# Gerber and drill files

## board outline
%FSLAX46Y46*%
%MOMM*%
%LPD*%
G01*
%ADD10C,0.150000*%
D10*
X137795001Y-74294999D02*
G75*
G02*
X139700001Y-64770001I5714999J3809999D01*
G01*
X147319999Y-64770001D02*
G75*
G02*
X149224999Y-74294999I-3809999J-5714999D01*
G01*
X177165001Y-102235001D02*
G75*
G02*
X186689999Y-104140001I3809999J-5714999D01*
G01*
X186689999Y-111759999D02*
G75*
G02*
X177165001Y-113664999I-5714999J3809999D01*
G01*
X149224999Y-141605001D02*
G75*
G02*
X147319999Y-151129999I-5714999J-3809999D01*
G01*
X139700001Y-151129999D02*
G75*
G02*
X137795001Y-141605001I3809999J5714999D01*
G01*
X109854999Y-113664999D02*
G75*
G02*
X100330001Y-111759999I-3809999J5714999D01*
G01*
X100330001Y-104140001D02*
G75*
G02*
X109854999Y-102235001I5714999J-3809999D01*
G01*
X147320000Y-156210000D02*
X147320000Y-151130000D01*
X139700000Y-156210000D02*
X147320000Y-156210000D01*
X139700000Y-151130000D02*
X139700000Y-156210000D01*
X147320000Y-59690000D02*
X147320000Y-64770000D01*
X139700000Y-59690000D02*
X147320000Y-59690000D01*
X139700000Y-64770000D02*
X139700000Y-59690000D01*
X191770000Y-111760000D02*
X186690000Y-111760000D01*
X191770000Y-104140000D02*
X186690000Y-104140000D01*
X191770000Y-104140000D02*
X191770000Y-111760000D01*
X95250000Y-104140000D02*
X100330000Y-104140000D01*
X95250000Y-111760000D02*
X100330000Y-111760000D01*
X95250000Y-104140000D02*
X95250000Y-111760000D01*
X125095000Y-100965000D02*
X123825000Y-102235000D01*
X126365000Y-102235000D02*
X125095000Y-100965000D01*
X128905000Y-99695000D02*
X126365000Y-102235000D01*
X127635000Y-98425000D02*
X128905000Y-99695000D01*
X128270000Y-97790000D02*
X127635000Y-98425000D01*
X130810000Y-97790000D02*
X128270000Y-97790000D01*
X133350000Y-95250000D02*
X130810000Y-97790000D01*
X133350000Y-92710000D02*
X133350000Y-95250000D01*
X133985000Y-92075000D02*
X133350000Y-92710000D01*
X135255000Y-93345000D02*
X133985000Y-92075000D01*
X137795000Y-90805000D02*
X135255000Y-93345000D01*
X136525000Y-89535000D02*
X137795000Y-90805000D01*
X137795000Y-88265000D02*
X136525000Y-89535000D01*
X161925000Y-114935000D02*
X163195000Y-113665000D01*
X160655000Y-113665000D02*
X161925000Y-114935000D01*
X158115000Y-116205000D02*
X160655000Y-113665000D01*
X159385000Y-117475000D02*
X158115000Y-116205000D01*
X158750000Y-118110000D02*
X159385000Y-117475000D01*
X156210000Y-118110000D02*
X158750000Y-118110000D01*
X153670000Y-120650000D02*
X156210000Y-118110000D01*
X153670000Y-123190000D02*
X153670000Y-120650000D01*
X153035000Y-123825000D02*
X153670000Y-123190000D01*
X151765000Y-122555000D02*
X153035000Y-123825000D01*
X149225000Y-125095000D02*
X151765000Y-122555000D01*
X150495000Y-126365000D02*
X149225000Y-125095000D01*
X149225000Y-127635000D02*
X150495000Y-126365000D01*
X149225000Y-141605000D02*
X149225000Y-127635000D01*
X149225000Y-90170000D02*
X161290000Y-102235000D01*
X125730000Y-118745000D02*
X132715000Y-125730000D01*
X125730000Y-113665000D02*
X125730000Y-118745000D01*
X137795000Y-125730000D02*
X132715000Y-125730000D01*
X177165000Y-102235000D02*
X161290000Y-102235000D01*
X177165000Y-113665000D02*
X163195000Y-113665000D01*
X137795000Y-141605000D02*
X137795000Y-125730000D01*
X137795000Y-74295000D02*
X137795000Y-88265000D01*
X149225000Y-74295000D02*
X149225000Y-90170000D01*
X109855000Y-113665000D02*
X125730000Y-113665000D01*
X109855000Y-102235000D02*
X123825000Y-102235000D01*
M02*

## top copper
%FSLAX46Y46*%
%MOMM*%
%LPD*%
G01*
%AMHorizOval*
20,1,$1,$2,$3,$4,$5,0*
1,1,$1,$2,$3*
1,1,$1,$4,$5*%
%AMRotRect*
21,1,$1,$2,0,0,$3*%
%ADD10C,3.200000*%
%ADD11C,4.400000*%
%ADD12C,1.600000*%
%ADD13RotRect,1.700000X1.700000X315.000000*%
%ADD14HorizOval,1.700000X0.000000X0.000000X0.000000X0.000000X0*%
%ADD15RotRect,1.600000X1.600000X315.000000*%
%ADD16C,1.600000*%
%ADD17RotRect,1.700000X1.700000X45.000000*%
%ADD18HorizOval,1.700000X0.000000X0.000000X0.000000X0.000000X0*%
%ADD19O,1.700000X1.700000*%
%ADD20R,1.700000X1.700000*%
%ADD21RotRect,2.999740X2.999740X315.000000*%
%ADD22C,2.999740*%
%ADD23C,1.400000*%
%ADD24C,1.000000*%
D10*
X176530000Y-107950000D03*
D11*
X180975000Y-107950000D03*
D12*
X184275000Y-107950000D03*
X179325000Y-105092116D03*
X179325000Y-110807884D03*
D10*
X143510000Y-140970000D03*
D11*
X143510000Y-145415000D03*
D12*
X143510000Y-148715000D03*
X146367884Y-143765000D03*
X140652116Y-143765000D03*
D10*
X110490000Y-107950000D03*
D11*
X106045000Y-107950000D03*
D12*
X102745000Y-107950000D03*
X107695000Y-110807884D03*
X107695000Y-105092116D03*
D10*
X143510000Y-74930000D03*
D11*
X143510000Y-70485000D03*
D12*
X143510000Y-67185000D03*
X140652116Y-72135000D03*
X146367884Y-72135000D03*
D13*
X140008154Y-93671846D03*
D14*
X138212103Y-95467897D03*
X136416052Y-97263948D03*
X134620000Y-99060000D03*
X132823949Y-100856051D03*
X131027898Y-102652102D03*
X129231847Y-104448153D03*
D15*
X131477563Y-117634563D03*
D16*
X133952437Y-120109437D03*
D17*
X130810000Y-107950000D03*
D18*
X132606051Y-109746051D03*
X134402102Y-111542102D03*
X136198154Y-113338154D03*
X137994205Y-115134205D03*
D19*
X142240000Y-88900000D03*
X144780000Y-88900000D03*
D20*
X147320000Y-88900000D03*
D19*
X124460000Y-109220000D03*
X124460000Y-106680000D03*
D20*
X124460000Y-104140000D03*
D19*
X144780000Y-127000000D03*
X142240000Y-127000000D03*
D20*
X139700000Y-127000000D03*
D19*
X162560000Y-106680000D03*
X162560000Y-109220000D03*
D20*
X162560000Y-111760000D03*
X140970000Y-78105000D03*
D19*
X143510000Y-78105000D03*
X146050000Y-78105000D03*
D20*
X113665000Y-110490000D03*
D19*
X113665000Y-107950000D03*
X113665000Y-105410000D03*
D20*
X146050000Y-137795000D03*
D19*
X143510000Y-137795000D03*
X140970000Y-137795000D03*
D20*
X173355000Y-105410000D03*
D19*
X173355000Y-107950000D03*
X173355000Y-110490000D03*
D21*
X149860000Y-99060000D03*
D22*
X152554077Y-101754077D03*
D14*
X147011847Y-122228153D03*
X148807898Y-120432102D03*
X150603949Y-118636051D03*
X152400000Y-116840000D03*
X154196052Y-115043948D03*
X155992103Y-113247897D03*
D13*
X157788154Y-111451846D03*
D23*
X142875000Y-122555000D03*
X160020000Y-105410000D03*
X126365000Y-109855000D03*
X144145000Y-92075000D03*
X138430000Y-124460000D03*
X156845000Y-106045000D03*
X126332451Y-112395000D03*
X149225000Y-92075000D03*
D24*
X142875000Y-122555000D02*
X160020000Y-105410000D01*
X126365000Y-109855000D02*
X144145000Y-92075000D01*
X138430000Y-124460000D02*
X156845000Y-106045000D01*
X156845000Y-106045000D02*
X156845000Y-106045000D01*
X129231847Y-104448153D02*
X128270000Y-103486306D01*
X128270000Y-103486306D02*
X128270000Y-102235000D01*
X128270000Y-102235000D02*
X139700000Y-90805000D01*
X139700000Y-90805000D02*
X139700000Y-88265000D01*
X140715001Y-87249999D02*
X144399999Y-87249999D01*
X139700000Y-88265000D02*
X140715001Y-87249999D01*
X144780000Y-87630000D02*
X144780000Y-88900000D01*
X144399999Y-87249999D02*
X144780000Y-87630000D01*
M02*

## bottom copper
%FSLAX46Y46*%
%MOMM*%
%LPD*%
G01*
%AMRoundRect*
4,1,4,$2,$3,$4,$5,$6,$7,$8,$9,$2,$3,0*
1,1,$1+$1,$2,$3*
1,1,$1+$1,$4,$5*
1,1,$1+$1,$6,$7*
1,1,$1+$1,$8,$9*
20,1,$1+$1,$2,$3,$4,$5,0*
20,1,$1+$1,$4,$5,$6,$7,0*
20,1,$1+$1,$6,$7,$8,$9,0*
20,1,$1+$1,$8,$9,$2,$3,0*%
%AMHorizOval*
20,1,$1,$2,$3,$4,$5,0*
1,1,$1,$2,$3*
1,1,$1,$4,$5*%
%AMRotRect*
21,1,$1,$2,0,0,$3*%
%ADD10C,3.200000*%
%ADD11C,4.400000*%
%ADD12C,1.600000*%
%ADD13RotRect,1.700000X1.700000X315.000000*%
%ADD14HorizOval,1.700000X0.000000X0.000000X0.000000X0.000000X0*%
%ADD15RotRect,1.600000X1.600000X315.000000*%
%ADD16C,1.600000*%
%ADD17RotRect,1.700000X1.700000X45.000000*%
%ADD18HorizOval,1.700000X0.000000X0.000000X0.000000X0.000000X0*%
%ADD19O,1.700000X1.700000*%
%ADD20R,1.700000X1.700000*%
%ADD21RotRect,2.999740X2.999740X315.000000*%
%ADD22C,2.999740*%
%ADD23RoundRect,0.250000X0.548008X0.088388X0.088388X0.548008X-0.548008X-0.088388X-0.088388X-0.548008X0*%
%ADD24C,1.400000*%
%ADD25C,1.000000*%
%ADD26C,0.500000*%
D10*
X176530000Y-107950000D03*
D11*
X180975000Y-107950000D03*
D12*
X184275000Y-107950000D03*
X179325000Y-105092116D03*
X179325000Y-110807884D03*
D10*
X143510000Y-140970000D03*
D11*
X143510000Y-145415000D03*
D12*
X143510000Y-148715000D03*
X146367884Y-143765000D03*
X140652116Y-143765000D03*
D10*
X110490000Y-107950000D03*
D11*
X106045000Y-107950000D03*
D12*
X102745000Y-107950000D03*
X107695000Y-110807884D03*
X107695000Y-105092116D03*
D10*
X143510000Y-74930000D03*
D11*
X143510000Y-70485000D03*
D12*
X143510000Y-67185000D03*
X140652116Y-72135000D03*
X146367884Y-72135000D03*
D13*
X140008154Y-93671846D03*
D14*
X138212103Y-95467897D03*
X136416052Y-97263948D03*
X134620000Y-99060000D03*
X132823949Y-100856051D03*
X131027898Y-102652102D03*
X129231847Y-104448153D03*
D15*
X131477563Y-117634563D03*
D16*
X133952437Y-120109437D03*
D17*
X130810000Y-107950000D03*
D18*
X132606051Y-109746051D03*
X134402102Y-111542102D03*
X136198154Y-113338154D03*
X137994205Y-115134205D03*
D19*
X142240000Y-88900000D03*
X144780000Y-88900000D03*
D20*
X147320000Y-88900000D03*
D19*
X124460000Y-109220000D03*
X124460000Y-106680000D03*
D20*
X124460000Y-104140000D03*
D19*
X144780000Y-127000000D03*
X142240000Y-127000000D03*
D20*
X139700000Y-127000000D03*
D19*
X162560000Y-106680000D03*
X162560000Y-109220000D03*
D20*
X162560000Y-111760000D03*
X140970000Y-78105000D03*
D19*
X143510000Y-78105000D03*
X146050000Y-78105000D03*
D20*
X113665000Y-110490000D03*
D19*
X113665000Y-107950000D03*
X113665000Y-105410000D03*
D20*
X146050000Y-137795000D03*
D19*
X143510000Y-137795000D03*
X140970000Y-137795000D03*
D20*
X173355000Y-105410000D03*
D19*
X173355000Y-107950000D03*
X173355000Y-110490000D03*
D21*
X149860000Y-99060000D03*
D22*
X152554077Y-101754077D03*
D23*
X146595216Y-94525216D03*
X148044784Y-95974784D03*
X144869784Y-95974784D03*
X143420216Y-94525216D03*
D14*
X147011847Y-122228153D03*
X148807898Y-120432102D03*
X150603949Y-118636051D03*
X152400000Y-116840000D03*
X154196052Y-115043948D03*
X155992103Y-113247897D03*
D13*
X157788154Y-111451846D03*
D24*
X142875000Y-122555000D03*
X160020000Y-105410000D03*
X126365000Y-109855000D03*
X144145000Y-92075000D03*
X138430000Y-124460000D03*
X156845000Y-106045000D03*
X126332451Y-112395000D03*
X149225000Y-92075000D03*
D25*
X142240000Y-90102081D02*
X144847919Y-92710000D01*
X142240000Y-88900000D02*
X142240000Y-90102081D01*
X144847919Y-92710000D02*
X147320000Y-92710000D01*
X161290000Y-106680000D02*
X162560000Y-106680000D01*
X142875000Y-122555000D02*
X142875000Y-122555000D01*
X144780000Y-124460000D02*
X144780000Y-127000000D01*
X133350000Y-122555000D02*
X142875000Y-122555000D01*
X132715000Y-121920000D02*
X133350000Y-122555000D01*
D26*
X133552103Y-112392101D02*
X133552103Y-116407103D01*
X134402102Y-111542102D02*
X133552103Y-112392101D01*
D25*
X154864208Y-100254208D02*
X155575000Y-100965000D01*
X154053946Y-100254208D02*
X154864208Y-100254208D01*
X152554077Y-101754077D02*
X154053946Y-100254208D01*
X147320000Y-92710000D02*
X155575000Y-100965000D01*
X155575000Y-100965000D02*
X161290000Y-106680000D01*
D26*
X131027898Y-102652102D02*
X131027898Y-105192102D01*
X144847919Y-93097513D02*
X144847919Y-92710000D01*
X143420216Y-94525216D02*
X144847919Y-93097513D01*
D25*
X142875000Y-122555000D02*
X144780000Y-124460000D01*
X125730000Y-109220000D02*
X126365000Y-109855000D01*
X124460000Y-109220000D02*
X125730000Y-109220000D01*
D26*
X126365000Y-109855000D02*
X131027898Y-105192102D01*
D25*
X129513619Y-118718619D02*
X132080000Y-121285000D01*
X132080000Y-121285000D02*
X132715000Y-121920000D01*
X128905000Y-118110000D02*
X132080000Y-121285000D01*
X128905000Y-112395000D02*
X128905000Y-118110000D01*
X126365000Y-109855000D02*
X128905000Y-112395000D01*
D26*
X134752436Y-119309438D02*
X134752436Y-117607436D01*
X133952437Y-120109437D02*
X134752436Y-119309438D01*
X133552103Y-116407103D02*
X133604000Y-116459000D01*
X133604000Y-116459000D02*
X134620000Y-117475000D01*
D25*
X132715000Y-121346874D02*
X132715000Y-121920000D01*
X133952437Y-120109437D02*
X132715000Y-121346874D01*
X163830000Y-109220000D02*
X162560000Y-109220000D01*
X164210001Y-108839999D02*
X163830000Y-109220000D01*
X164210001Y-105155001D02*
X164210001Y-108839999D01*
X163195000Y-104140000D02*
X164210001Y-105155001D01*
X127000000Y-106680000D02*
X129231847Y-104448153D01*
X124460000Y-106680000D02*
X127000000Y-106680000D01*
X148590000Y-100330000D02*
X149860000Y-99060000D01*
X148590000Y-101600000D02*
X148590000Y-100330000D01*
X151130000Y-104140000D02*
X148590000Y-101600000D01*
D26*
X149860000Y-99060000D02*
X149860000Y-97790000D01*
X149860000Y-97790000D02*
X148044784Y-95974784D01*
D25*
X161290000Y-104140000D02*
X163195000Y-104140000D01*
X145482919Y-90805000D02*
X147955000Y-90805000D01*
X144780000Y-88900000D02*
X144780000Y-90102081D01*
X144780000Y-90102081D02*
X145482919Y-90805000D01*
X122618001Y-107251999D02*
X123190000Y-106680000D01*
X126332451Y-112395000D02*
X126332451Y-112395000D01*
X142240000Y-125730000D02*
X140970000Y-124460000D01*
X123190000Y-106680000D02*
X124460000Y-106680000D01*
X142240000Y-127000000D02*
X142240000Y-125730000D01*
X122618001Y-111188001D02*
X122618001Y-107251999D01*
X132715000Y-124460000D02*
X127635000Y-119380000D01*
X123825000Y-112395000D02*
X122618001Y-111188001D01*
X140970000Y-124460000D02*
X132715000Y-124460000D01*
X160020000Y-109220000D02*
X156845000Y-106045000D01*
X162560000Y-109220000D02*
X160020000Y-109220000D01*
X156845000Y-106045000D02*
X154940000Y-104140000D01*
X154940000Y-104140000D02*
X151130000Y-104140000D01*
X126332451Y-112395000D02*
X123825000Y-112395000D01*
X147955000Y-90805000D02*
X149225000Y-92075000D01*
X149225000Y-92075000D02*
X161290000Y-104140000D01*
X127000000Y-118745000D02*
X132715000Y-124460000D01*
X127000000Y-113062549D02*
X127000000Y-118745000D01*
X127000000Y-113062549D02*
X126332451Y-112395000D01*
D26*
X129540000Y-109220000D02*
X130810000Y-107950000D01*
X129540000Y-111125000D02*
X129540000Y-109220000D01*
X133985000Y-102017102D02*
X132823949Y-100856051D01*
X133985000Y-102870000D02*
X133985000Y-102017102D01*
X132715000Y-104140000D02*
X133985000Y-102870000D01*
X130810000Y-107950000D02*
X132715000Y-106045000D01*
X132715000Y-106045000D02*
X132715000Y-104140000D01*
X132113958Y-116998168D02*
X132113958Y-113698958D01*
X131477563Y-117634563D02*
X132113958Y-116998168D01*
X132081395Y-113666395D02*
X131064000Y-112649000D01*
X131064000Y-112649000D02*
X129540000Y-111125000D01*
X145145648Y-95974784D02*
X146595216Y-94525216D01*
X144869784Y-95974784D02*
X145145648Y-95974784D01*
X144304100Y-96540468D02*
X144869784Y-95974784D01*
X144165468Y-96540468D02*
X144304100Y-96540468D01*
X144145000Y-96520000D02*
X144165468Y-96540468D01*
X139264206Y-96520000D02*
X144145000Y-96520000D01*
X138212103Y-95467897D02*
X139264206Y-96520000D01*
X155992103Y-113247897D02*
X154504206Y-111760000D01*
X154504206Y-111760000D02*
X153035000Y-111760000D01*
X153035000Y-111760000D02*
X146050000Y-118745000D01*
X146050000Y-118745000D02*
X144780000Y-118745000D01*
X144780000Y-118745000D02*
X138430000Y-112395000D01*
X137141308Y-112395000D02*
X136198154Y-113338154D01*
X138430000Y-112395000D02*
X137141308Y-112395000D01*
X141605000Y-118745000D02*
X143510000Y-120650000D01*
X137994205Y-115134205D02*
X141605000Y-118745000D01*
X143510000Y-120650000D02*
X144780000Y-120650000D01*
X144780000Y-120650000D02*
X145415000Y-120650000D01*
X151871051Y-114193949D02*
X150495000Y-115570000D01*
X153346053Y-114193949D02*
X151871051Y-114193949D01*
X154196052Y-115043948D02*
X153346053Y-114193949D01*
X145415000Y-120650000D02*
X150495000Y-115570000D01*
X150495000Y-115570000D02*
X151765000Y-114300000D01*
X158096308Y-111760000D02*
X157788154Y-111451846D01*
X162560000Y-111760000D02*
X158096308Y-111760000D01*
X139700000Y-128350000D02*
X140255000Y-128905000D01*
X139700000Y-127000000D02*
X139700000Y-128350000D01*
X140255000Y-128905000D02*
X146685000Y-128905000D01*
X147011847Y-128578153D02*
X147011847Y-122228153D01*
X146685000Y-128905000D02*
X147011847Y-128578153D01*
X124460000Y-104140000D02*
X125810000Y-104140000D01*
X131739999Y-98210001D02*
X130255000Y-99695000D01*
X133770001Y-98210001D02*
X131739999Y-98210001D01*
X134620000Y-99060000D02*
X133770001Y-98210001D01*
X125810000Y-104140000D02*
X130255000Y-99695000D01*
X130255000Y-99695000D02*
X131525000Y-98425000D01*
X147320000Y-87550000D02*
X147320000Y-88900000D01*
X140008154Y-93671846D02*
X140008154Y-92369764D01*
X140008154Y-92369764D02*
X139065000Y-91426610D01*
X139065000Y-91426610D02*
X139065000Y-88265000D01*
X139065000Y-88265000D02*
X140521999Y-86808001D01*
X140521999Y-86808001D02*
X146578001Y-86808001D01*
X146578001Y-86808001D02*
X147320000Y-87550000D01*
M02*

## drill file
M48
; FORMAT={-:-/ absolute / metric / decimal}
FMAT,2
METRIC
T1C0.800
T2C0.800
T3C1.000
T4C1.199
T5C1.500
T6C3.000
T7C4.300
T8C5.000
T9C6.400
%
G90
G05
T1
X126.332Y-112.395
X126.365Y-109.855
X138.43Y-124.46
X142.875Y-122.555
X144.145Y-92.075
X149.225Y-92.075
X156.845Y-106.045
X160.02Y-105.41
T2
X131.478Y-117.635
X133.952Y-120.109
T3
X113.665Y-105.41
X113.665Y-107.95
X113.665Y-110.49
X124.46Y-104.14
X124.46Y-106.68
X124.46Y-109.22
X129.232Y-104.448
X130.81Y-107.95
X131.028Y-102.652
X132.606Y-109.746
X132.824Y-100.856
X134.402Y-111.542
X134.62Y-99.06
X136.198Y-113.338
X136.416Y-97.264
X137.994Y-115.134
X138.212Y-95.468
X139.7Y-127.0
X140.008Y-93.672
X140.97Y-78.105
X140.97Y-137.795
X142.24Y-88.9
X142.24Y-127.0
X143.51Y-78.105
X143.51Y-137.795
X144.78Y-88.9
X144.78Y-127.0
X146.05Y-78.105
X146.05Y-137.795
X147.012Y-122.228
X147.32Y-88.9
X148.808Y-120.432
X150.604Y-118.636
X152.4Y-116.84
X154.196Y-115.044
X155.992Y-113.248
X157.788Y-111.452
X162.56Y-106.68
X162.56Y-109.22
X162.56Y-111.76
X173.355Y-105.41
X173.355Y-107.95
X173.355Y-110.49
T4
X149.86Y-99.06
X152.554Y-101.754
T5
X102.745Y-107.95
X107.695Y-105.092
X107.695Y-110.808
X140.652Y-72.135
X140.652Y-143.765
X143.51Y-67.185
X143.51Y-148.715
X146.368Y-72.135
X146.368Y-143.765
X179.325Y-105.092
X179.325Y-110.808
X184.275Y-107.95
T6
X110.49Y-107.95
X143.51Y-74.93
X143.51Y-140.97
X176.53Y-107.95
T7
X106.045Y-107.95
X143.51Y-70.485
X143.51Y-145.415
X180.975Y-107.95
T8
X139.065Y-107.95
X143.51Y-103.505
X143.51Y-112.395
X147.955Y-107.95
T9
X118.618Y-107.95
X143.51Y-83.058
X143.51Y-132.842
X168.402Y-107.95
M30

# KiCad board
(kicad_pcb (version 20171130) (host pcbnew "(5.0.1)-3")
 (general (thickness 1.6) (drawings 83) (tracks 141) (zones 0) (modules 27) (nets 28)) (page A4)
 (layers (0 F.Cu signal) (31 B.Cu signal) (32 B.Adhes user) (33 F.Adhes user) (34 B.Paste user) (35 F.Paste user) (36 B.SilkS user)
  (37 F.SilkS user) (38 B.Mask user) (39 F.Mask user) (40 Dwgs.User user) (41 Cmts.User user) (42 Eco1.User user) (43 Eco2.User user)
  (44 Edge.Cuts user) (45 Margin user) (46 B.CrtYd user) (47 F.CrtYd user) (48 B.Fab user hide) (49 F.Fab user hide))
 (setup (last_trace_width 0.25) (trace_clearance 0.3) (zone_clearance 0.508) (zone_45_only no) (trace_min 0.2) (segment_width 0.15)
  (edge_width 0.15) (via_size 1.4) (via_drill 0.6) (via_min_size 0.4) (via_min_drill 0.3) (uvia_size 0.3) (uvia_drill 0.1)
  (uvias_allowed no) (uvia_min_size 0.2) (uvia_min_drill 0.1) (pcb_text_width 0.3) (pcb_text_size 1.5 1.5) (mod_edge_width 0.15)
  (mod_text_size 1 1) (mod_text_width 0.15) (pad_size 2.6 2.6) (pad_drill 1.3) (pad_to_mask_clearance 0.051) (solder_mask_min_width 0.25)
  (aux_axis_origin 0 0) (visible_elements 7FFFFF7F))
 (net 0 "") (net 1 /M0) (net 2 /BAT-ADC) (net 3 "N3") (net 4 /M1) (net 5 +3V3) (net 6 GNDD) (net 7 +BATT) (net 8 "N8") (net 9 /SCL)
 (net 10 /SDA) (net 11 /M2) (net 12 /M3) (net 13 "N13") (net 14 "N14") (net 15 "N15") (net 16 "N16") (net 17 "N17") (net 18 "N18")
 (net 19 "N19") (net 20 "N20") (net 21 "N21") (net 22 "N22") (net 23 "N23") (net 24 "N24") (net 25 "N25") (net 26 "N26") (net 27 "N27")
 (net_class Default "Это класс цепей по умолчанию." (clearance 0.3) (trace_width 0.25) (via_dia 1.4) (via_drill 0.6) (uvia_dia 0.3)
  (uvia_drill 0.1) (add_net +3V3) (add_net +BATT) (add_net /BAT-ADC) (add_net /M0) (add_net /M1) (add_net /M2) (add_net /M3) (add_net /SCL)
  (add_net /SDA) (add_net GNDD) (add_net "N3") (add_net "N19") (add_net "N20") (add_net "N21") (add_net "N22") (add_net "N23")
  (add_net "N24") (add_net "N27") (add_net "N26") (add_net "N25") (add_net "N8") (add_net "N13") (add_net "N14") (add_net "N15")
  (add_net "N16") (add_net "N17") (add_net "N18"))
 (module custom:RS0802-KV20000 (layer F.Cu) (at 180.975 107.95)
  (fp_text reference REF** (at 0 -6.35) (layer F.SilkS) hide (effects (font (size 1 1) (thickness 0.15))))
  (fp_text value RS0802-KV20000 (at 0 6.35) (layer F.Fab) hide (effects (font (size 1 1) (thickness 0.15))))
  (pad "" np_thru_hole circle (at -4.445 0) (size 3.2 3.2) (drill 3) (layers *.Cu *.Mask))
  (pad "" np_thru_hole circle (at 0 0) (size 4.4 4.4) (drill 4.3) (layers *.Cu *.Mask))
  (pad "" np_thru_hole circle (at 3.3 0) (size 1.6 1.6) (drill 1.5) (layers *.Cu *.Mask))
  (pad "" np_thru_hole circle (at -1.65 -2.857884 120) (size 1.6 1.6) (drill 1.5) (layers *.Cu *.Mask))
  (pad "" np_thru_hole circle (at -1.65 2.857884 240) (size 1.6 1.6) (drill 1.5) (layers *.Cu *.Mask)))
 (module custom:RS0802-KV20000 (layer F.Cu) (at 143.51 145.415 270)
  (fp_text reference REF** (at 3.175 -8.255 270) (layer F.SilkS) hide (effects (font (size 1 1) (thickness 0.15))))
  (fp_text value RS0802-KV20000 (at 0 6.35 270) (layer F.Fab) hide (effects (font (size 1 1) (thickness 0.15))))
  (pad "" np_thru_hole circle (at -4.445 0 270) (size 3.2 3.2) (drill 3) (layers *.Cu *.Mask))
  (pad "" np_thru_hole circle (at 0 0 270) (size 4.4 4.4) (drill 4.3) (layers *.Cu *.Mask))
  (pad "" np_thru_hole circle (at 3.3 0 270) (size 1.6 1.6) (drill 1.5) (layers *.Cu *.Mask))
  (pad "" np_thru_hole circle (at -1.65 -2.857884 30) (size 1.6 1.6) (drill 1.5) (layers *.Cu *.Mask))
  (pad "" np_thru_hole circle (at -1.65 2.857884 150) (size 1.6 1.6) (drill 1.5) (layers *.Cu *.Mask)))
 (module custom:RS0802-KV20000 (layer F.Cu) (at 106.045 107.95 180)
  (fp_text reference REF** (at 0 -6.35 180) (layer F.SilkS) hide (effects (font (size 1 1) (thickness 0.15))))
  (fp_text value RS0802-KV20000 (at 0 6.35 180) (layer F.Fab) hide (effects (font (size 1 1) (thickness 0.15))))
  (pad "" np_thru_hole circle (at -4.445 0 180) (size 3.2 3.2) (drill 3) (layers *.Cu *.Mask))
  (pad "" np_thru_hole circle (at 0 0 180) (size 4.4 4.4) (drill 4.3) (layers *.Cu *.Mask))
  (pad "" np_thru_hole circle (at 3.3 0 180) (size 1.6 1.6) (drill 1.5) (layers *.Cu *.Mask))
  (pad "" np_thru_hole circle (at -1.65 -2.857884 300) (size 1.6 1.6) (drill 1.5) (layers *.Cu *.Mask))
  (pad "" np_thru_hole circle (at -1.65 2.857884 60) (size 1.6 1.6) (drill 1.5) (layers *.Cu *.Mask)))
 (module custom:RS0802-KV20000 (layer F.Cu) (at 143.51 70.485 90)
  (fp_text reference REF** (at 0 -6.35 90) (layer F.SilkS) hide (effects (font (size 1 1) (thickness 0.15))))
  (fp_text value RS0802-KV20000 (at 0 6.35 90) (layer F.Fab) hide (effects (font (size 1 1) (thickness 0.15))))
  (pad "" np_thru_hole circle (at -4.445 0 90) (size 3.2 3.2) (drill 3) (layers *.Cu *.Mask))
  (pad "" np_thru_hole circle (at 0 0 90) (size 4.4 4.4) (drill 4.3) (layers *.Cu *.Mask))
  (pad "" np_thru_hole circle (at 3.3 0 90) (size 1.6 1.6) (drill 1.5) (layers *.Cu *.Mask))
  (pad "" np_thru_hole circle (at -1.65 -2.857884 210) (size 1.6 1.6) (drill 1.5) (layers *.Cu *.Mask))
  (pad "" np_thru_hole circle (at -1.65 2.857884 330) (size 1.6 1.6) (drill 1.5) (layers *.Cu *.Mask)))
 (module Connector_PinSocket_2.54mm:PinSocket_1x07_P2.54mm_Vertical (layer F.Cu) (at 140.008154 93.671846 315)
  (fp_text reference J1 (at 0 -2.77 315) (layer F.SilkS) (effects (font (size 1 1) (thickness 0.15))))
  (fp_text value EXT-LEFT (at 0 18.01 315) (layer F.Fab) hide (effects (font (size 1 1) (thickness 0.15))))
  (pad 1 thru_hole rect (at 0 0 315) (size 1.7 1.7) (drill 1) (layers *.Cu *.Mask) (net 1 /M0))
  (pad 2 thru_hole oval (at 0 2.54 315) (size 1.7 1.7) (drill 1) (layers *.Cu *.Mask) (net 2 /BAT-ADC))
  (pad 3 thru_hole oval (at 0 5.079999 315) (size 1.7 1.7) (drill 1) (layers *.Cu *.Mask) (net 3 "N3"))
  (pad 4 thru_hole oval (at 0 7.62 315) (size 1.7 1.7) (drill 1) (layers *.Cu *.Mask) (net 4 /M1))
  (pad 5 thru_hole oval (at 0 10.16 315) (size 1.7 1.7) (drill 1) (layers *.Cu *.Mask) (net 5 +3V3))
  (pad 6 thru_hole oval (at 0 12.7 315) (size 1.7 1.7) (drill 1) (layers *.Cu *.Mask) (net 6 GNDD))
  (pad 7 thru_hole oval (at 0 15.24 315) (size 1.7 1.7) (drill 1) (layers *.Cu *.Mask) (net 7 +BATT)))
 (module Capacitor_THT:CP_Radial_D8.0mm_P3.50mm (layer F.Cu) (at 132.715 118.872 315)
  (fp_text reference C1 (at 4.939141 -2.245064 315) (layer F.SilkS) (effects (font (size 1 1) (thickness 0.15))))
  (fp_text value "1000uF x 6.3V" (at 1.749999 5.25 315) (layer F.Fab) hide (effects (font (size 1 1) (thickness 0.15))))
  (pad 1 thru_hole rect (at -1.75 0 315) (size 1.6 1.6) (drill 0.8) (layers *.Cu *.Mask) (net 5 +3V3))
  (pad 2 thru_hole circle (at 1.75 0 315) (size 1.6 1.6) (drill 0.8) (layers *.Cu *.Mask) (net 6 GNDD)))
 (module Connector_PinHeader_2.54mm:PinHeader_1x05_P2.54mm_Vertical (layer F.Cu) (at 130.81 107.95 45)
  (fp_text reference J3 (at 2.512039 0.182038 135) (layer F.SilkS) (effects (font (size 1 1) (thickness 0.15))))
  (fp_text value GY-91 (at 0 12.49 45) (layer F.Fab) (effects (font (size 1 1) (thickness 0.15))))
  (pad 1 thru_hole rect (at 0 0 45) (size 1.7 1.7) (drill 1) (layers *.Cu *.Mask) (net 5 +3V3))
  (pad 2 thru_hole oval (at 0 2.54 45) (size 1.7 1.7) (drill 1) (layers *.Cu *.Mask) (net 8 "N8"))
  (pad 3 thru_hole oval (at 0 5.079999 45) (size 1.7 1.7) (drill 1) (layers *.Cu *.Mask) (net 6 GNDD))
  (pad 4 thru_hole oval (at 0 7.62 45) (size 1.7 1.7) (drill 1) (layers *.Cu *.Mask) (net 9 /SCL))
  (pad 5 thru_hole oval (at 0 10.16 45) (size 1.7 1.7) (drill 1) (layers *.Cu *.Mask) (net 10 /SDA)))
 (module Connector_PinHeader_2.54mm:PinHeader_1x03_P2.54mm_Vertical (layer F.Cu) (at 147.32 88.9 270)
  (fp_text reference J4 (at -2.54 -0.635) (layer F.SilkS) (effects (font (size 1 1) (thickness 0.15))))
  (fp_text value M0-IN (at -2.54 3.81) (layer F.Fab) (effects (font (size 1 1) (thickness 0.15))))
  (pad 3 thru_hole oval (at 0 5.08 270) (size 1.7 1.7) (drill 1) (layers *.Cu *.Mask) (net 6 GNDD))
  (pad 2 thru_hole oval (at 0 2.54 270) (size 1.7 1.7) (drill 1) (layers *.Cu *.Mask) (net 7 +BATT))
  (pad 1 thru_hole rect (at 0 0 270) (size 1.7 1.7) (drill 1) (layers *.Cu *.Mask) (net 1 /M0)))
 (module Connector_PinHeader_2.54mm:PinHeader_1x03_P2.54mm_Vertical (layer F.Cu) (at 124.46 104.14)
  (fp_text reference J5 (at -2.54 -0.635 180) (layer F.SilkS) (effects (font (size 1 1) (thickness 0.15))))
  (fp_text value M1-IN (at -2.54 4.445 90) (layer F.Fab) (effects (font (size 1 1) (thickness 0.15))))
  (pad 3 thru_hole oval (at 0 5.08) (size 1.7 1.7) (drill 1) (layers *.Cu *.Mask) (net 6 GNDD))
  (pad 2 thru_hole oval (at 0 2.54) (size 1.7 1.7) (drill 1) (layers *.Cu *.Mask) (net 7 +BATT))
  (pad 1 thru_hole rect (at 0 0) (size 1.7 1.7) (drill 1) (layers *.Cu *.Mask) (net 4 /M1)))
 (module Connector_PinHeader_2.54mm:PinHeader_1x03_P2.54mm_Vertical (layer F.Cu) (at 139.7 127 90)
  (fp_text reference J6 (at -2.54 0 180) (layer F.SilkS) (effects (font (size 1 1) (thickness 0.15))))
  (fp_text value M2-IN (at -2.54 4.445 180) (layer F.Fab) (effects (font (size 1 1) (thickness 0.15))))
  (pad 3 thru_hole oval (at 0 5.08 90) (size 1.7 1.7) (drill 1) (layers *.Cu *.Mask) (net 6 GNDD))
  (pad 2 thru_hole oval (at 0 2.54 90) (size 1.7 1.7) (drill 1) (layers *.Cu *.Mask) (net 7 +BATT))
  (pad 1 thru_hole rect (at 0 0 90) (size 1.7 1.7) (drill 1) (layers *.Cu *.Mask) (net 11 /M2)))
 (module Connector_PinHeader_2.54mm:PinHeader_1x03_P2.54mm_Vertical (layer F.Cu) (at 162.56 111.76 180)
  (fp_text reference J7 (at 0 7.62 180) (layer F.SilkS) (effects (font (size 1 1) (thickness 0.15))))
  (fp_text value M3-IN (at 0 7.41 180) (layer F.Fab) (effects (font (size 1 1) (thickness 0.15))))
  (pad 3 thru_hole oval (at 0 5.08 180) (size 1.7 1.7) (drill 1) (layers *.Cu *.Mask) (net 6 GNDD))
  (pad 2 thru_hole oval (at 0 2.54 180) (size 1.7 1.7) (drill 1) (layers *.Cu *.Mask) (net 7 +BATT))
  (pad 1 thru_hole rect (at 0 0 180) (size 1.7 1.7) (drill 1) (layers *.Cu *.Mask) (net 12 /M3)))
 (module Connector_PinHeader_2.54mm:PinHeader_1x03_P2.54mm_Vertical (layer F.Cu) (at 140.97 78.105 90)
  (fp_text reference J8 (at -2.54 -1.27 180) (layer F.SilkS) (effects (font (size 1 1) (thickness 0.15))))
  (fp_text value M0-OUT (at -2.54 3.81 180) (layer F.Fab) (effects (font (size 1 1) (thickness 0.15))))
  (pad 1 thru_hole rect (at 0 0 90) (size 1.7 1.7) (drill 1) (layers *.Cu *.Mask) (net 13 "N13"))
  (pad 2 thru_hole oval (at 0 2.54 90) (size 1.7 1.7) (drill 1) (layers *.Cu *.Mask) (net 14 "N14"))
  (pad 3 thru_hole oval (at 0 5.08 90) (size 1.7 1.7) (drill 1) (layers *.Cu *.Mask) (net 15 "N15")))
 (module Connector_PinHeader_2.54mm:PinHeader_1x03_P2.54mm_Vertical (layer F.Cu) (at 113.665 110.49 180)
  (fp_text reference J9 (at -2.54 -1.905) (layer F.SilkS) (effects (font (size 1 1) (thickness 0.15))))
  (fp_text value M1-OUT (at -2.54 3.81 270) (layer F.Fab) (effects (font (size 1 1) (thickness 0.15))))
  (pad 1 thru_hole rect (at 0 0 180) (size 1.7 1.7) (drill 1) (layers *.Cu *.Mask) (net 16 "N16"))
  (pad 2 thru_hole oval (at 0 2.54 180) (size 1.7 1.7) (drill 1) (layers *.Cu *.Mask) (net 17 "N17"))
  (pad 3 thru_hole oval (at 0 5.08 180) (size 1.7 1.7) (drill 1) (layers *.Cu *.Mask) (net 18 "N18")))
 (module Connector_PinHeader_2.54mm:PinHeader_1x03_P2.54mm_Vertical (layer F.Cu) (at 146.05 137.795 270)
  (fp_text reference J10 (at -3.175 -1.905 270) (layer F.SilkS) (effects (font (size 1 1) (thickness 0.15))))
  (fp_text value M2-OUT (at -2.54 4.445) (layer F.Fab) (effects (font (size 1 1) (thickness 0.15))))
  (pad 1 thru_hole rect (at 0 0 270) (size 1.7 1.7) (drill 1) (layers *.Cu *.Mask) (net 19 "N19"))
  (pad 2 thru_hole oval (at 0 2.54 270) (size 1.7 1.7) (drill 1) (layers *.Cu *.Mask) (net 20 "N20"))
  (pad 3 thru_hole oval (at 0 5.08 270) (size 1.7 1.7) (drill 1) (layers *.Cu *.Mask) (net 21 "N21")))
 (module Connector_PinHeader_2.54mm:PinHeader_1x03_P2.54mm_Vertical (layer F.Cu) (at 173.355 105.41)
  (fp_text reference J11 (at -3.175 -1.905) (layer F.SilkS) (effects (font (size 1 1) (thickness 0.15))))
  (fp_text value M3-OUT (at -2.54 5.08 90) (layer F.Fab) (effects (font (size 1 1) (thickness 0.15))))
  (pad 1 thru_hole rect (at 0 0) (size 1.7 1.7) (drill 1) (layers *.Cu *.Mask) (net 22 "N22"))
  (pad 2 thru_hole oval (at 0 2.54) (size 1.7 1.7) (drill 1) (layers *.Cu *.Mask) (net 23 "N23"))
  (pad 3 thru_hole oval (at 0 5.08) (size 1.7 1.7) (drill 1) (layers *.Cu *.Mask) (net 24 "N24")))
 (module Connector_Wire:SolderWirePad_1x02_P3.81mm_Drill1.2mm (layer F.Cu) (at 149.86 99.06 315)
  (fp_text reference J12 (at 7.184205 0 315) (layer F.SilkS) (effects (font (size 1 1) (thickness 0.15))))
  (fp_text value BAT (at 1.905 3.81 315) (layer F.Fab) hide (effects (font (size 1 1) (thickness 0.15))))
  (pad 1 thru_hole rect (at 0 0 315) (size 2.99974 2.99974) (drill 1.19888) (layers *.Cu *.Mask) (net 7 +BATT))
  (pad 2 thru_hole circle (at 3.81 0 315) (size 2.99974 2.99974) (drill 1.19888) (layers *.Cu *.Mask) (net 6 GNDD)))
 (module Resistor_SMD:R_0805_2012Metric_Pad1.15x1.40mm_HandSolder (layer B.Cu) (at 147.32 95.25 135)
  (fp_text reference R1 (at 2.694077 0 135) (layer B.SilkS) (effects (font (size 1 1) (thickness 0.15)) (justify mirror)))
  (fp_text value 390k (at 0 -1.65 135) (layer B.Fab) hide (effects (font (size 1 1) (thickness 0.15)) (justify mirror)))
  (pad 2 smd roundrect (at 1.024999 0 135) (size 1.15 1.4) (layers B.Cu B.Paste B.Mask) (roundrect_rratio 0.217391) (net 2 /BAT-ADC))
  (pad 1 smd roundrect (at -1.024999 0 135) (size 1.15 1.4) (layers B.Cu B.Paste B.Mask) (roundrect_rratio 0.217391) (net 7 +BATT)))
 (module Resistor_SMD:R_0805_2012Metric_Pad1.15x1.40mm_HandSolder (layer B.Cu) (at 144.145 95.25 135)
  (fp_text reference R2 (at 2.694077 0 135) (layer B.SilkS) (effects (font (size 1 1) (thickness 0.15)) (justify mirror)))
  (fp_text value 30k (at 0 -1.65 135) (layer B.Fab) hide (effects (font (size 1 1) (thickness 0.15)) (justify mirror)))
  (pad 1 smd roundrect (at -1.024999 0 135) (size 1.15 1.4) (layers B.Cu B.Paste B.Mask) (roundrect_rratio 0.217391) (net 2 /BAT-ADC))
  (pad 2 smd roundrect (at 1.024999 0 135) (size 1.15 1.4) (layers B.Cu B.Paste B.Mask) (roundrect_rratio 0.217391) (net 6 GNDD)))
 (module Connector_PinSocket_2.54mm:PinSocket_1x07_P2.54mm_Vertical (layer F.Cu) (at 157.788154 111.451846 315)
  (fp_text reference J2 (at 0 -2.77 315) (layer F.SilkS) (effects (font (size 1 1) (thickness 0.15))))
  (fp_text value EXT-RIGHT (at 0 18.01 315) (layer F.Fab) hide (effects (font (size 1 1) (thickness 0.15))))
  (pad 7 thru_hole oval (at 0 15.24 315) (size 1.7 1.7) (drill 1) (layers *.Cu *.Mask) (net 11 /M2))
  (pad 6 thru_hole oval (at 0 12.7 315) (size 1.7 1.7) (drill 1) (layers *.Cu *.Mask) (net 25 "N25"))
  (pad 5 thru_hole oval (at 0 10.16 315) (size 1.7 1.7) (drill 1) (layers *.Cu *.Mask) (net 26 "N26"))
  (pad 4 thru_hole oval (at 0 7.62 315) (size 1.7 1.7) (drill 1) (layers *.Cu *.Mask) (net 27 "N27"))
  (pad 3 thru_hole oval (at 0 5.079999 315) (size 1.7 1.7) (drill 1) (layers *.Cu *.Mask) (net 10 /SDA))
  (pad 2 thru_hole oval (at 0 2.54 315) (size 1.7 1.7) (drill 1) (layers *.Cu *.Mask) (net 9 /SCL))
  (pad 1 thru_hole rect (at 0 0 315) (size 1.7 1.7) (drill 1) (layers *.Cu *.Mask) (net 12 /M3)))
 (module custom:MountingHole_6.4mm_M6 (layer F.Cu) (at 118.618 107.95)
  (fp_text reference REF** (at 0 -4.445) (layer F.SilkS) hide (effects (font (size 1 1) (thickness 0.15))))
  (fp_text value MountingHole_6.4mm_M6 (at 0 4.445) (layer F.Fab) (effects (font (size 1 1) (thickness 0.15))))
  (pad 1 np_thru_hole circle (at 0 0) (size 6.4 6.4) (drill 6.4) (layers *.Cu *.Mask)))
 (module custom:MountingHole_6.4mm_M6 (layer F.Cu) (at 143.51 132.842)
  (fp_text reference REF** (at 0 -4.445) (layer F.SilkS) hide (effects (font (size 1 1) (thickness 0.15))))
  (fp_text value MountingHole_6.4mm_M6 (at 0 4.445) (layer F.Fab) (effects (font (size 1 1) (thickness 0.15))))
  (pad 1 np_thru_hole circle (at 0 0) (size 6.4 6.4) (drill 6.4) (layers *.Cu *.Mask)))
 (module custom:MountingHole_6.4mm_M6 (layer F.Cu) (at 168.402 107.95)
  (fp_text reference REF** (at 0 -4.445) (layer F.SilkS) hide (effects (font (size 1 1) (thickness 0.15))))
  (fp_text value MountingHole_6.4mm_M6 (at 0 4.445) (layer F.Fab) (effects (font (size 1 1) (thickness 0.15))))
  (pad 1 np_thru_hole circle (at 0 0) (size 6.4 6.4) (drill 6.4) (layers *.Cu *.Mask)))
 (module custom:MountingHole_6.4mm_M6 (layer F.Cu) (at 143.51 83.058)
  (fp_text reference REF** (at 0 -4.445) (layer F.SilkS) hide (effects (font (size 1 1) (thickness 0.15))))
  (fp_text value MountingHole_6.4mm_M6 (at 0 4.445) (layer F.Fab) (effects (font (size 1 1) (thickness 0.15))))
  (pad 1 np_thru_hole circle (at 0 0) (size 6.4 6.4) (drill 6.4) (layers *.Cu *.Mask)))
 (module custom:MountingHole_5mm (layer F.Cu) (at 143.51 112.395)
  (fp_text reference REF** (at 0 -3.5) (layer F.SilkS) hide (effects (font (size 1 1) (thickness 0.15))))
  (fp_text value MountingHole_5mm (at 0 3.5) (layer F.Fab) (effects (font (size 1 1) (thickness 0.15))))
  (pad "" np_thru_hole circle (at 0 0) (size 5 5) (drill 5) (layers *.Cu *.Mask)))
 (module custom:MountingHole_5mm (layer F.Cu) (at 139.065 107.95)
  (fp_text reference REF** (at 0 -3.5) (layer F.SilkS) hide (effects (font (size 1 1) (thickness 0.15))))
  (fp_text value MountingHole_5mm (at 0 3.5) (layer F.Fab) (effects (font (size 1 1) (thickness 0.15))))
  (pad "" np_thru_hole circle (at 0 0) (size 5 5) (drill 5) (layers *.Cu *.Mask)))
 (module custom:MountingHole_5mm (layer F.Cu) (at 143.51 103.505)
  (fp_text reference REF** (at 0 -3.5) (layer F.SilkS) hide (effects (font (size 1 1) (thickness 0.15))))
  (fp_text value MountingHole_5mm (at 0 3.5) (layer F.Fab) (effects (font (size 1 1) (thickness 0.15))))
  (pad "" np_thru_hole circle (at 0 0) (size 5 5) (drill 5) (layers *.Cu *.Mask)))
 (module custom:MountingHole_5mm (layer F.Cu) (at 147.955 107.95)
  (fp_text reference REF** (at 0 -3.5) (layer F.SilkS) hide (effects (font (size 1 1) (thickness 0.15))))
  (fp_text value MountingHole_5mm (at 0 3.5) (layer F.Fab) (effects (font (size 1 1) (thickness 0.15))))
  (pad "" np_thru_hole circle (at 0 0) (size 5 5) (drill 5) (layers *.Cu *.Mask)))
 (gr_arc (start 143.51 70.485) (end 139.700001 64.770001) (angle -90) (layer Edge.Cuts) (width 0.15))
 (gr_arc (start 143.51 70.485) (end 149.224999 74.294999) (angle -90) (layer Edge.Cuts) (width 0.15))
 (gr_arc (start 180.975 107.95) (end 186.689999 104.140001) (angle -90) (layer Edge.Cuts) (width 0.15))
 (gr_arc (start 180.975 107.95) (end 177.165001 113.664999) (angle -90) (layer Edge.Cuts) (width 0.15))
 (gr_arc (start 143.51 145.415) (end 147.319999 151.129999) (angle -90) (layer Edge.Cuts) (width 0.15))
 (gr_arc (start 143.51 145.415) (end 137.795001 141.605001) (angle -90) (layer Edge.Cuts) (width 0.15))
 (gr_arc (start 106.045 107.95) (end 100.330001 111.759999) (angle -90) (layer Edge.Cuts) (width 0.15))
 (gr_arc (start 106.045 107.95) (end 109.854999 102.235001) (angle -90) (layer Edge.Cuts) (width 0.15))
 (gr_line (start 147.32 156.21) (end 147.32 151.13) (layer Edge.Cuts) (width 0.15))
 (gr_line (start 139.7 156.21) (end 147.32 156.21) (layer Edge.Cuts) (width 0.15))
 (gr_line (start 139.7 151.13) (end 139.7 156.21) (layer Edge.Cuts) (width 0.15))
 (gr_line (start 147.32 59.69) (end 147.32 64.77) (layer Edge.Cuts) (width 0.15))
 (gr_line (start 139.7 59.69) (end 147.32 59.69) (layer Edge.Cuts) (width 0.15))
 (gr_line (start 139.7 64.77) (end 139.7 59.69) (layer Edge.Cuts) (width 0.15))
 (gr_line (start 191.77 111.76) (end 186.69 111.76) (layer Edge.Cuts) (width 0.15))
 (gr_line (start 191.77 104.14) (end 186.69 104.14) (layer Edge.Cuts) (width 0.15))
 (gr_line (start 191.77 104.14) (end 191.77 111.76) (layer Edge.Cuts) (width 0.15))
 (gr_line (start 95.25 104.14) (end 100.33 104.14) (layer Edge.Cuts) (width 0.15))
 (gr_line (start 95.25 111.76) (end 100.33 111.76) (layer Edge.Cuts) (width 0.15))
 (gr_line (start 95.25 104.14) (end 95.25 111.76) (layer Edge.Cuts) (width 0.15))
 (gr_line (start 125.095 100.965) (end 123.825 102.235) (layer Edge.Cuts) (width 0.15))
 (gr_line (start 126.365 102.235) (end 125.095 100.965) (layer Edge.Cuts) (width 0.15))
 (gr_line (start 128.905 99.695) (end 126.365 102.235) (layer Edge.Cuts) (width 0.15))
 (gr_line (start 127.635 98.425) (end 128.905 99.695) (layer Edge.Cuts) (width 0.15))
 (gr_line (start 128.27 97.79) (end 127.635 98.425) (layer Edge.Cuts) (width 0.15))
 (gr_line (start 130.81 97.79) (end 128.27 97.79) (layer Edge.Cuts) (width 0.15))
 (gr_line (start 133.35 95.25) (end 130.81 97.79) (layer Edge.Cuts) (width 0.15))
 (gr_line (start 133.35 92.71) (end 133.35 95.25) (layer Edge.Cuts) (width 0.15))
 (gr_line (start 133.985 92.075) (end 133.35 92.71) (layer Edge.Cuts) (width 0.15))
 (gr_line (start 135.255 93.345) (end 133.985 92.075) (layer Edge.Cuts) (width 0.15))
 (gr_line (start 137.795 90.805) (end 135.255 93.345) (layer Edge.Cuts) (width 0.15))
 (gr_line (start 136.525 89.535) (end 137.795 90.805) (layer Edge.Cuts) (width 0.15))
 (gr_line (start 137.795 88.265) (end 136.525 89.535) (layer Edge.Cuts) (width 0.15))
 (gr_line (start 161.925 114.935) (end 163.195 113.665) (layer Edge.Cuts) (width 0.15))
 (gr_line (start 160.655 113.665) (end 161.925 114.935) (layer Edge.Cuts) (width 0.15))
 (gr_line (start 158.115 116.205) (end 160.655 113.665) (layer Edge.Cuts) (width 0.15))
 (gr_line (start 159.385 117.475) (end 158.115 116.205) (layer Edge.Cuts) (width 0.15))
 (gr_line (start 158.75 118.11) (end 159.385 117.475) (layer Edge.Cuts) (width 0.15))
 (gr_line (start 156.21 118.11) (end 158.75 118.11) (layer Edge.Cuts) (width 0.15))
 (gr_line (start 153.67 120.65) (end 156.21 118.11) (layer Edge.Cuts) (width 0.15))
 (gr_line (start 153.67 123.19) (end 153.67 120.65) (layer Edge.Cuts) (width 0.15))
 (gr_line (start 153.035 123.825) (end 153.67 123.19) (layer Edge.Cuts) (width 0.15))
 (gr_line (start 151.765 122.555) (end 153.035 123.825) (layer Edge.Cuts) (width 0.15))
 (gr_line (start 149.225 125.095) (end 151.765 122.555) (layer Edge.Cuts) (width 0.15))
 (gr_line (start 150.495 126.365) (end 149.225 125.095) (layer Edge.Cuts) (width 0.15))
 (gr_line (start 149.225 127.635) (end 150.495 126.365) (layer Edge.Cuts) (width 0.15))
 (gr_line (start 149.225 141.605) (end 149.225 127.635) (layer Edge.Cuts) (width 0.15))
 (gr_line (start 149.225 90.17) (end 161.29 102.235) (layer Edge.Cuts) (width 0.15))
 (gr_line (start 125.73 118.745) (end 132.715 125.73) (layer Edge.Cuts) (width 0.15))
 (gr_line (start 125.73 113.665) (end 125.73 118.745) (layer Edge.Cuts) (width 0.15))
 (gr_line (start 137.795 125.73) (end 132.715 125.73) (layer Edge.Cuts) (width 0.15))
 (gr_line (start 177.165 102.235) (end 161.29 102.235) (layer Edge.Cuts) (width 0.15))
 (gr_line (start 177.165 113.665) (end 163.195 113.665) (layer Edge.Cuts) (width 0.15))
 (gr_line (start 137.795 141.605) (end 137.795 125.73) (layer Edge.Cuts) (width 0.15))
 (gr_line (start 137.795 74.295) (end 137.795 88.265) (layer Edge.Cuts) (width 0.15))
 (gr_line (start 149.225 74.295) (end 149.225 90.17) (layer Edge.Cuts) (width 0.15))
 (gr_line (start 109.855 113.665) (end 125.73 113.665) (layer Edge.Cuts) (width 0.15))
 (gr_line (start 109.855 102.235) (end 123.825 102.235) (layer Edge.Cuts) (width 0.15))
 (segment (start 142.24 90.102081) (end 144.847919 92.71) (width 1) (layer B.Cu) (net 6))
 (segment (start 142.24 88.9) (end 142.24 90.102081) (width 1) (layer B.Cu) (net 6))
 (segment (start 144.847919 92.71) (end 147.32 92.71) (width 1) (layer B.Cu) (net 6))
 (segment (start 161.29 106.68) (end 162.56 106.68) (width 1) (layer B.Cu) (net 6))
 (segment (start 142.875 122.555) (end 142.875 122.555) (width 1) (layer B.Cu) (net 6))
 (segment (start 144.78 124.46) (end 144.78 127) (width 1) (layer B.Cu) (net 6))
 (segment (start 133.35 122.555) (end 142.875 122.555) (width 1) (layer B.Cu) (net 6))
 (segment (start 132.715 121.92) (end 133.35 122.555) (width 1) (layer B.Cu) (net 6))
 (segment (start 133.552103 112.392101) (end 133.552103 116.407103) (width 0.5) (layer B.Cu) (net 6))
 (segment (start 134.402102 111.542102) (end 133.552103 112.392101) (width 0.5) (layer B.Cu) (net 6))
 (segment (start 154.864208 100.254208) (end 155.575 100.965) (width 1) (layer B.Cu) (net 6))
 (segment (start 154.053946 100.254208) (end 154.864208 100.254208) (width 1) (layer B.Cu) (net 6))
 (segment (start 152.554077 101.754077) (end 154.053946 100.254208) (width 1) (layer B.Cu) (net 6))
 (segment (start 147.32 92.71) (end 155.575 100.965) (width 1) (layer B.Cu) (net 6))
 (segment (start 155.575 100.965) (end 161.29 106.68) (width 1) (layer B.Cu) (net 6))
 (segment (start 131.027898 102.652102) (end 131.027898 105.192102) (width 0.5) (layer B.Cu) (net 6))
 (segment (start 144.847919 93.097513) (end 144.847919 92.71) (width 0.5) (layer B.Cu) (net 6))
 (segment (start 143.420216 94.525216) (end 144.847919 93.097513) (width 0.5) (layer B.Cu) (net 6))
 (segment (start 142.875 122.555) (end 144.78 124.46) (width 1) (layer B.Cu) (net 6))
 (via (at 142.875 122.555) (size 1.4) (drill 0.8) (layers F.Cu B.Cu) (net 6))
 (segment (start 142.875 122.555) (end 160.02 105.41) (width 1) (layer F.Cu) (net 6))
 (via (at 160.02 105.41) (size 1.4) (drill 0.8) (layers F.Cu B.Cu) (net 6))
 (via (at 126.365 109.855) (size 1.4) (drill 0.8) (layers F.Cu B.Cu) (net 6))
 (segment (start 125.73 109.22) (end 126.365 109.855) (width 1) (layer B.Cu) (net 6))
 (segment (start 124.46 109.22) (end 125.73 109.22) (width 1) (layer B.Cu) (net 6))
 (segment (start 126.365 109.855) (end 131.027898 105.192102) (width 0.5) (layer B.Cu) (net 6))
 (via (at 144.145 92.075) (size 1.4) (drill 0.8) (layers F.Cu B.Cu) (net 6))
 (segment (start 126.365 109.855) (end 144.145 92.075) (width 1) (layer F.Cu) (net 6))
 (segment (start 129.513619 118.718619) (end 132.08 121.285) (width 1) (layer B.Cu) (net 6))
 (segment (start 132.08 121.285) (end 132.715 121.92) (width 1) (layer B.Cu) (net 6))
 (segment (start 128.905 118.11) (end 132.08 121.285) (width 1) (layer B.Cu) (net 6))
 (segment (start 128.905 112.395) (end 128.905 118.11) (width 1) (layer B.Cu) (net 6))
 (segment (start 126.365 109.855) (end 128.905 112.395) (width 1) (layer B.Cu) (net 6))
 (segment (start 134.752436 119.309438) (end 134.752436 117.607436) (width 0.5) (layer B.Cu) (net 6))
 (segment (start 133.952437 120.109437) (end 134.752436 119.309438) (width 0.5) (layer B.Cu) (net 6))
 (segment (start 133.552103 116.407103) (end 133.604 116.459) (width 0.5) (layer B.Cu) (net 6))
 (segment (start 133.604 116.459) (end 134.62 117.475) (width 0.5) (layer B.Cu) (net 6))
 (segment (start 132.715 121.346874) (end 132.715 121.92) (width 1) (layer B.Cu) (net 6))
 (segment (start 133.952437 120.109437) (end 132.715 121.346874) (width 1) (layer B.Cu) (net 6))
 (segment (start 163.83 109.22) (end 162.56 109.22) (width 1) (layer B.Cu) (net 7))
 (segment (start 164.210001 108.839999) (end 163.83 109.22) (width 1) (layer B.Cu) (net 7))
 (segment (start 164.210001 105.155001) (end 164.210001 108.839999) (width 1) (layer B.Cu) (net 7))
 (segment (start 163.195 104.14) (end 164.210001 105.155001) (width 1) (layer B.Cu) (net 7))
 (segment (start 127 106.68) (end 129.231847 104.448153) (width 1) (layer B.Cu) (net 7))
 (segment (start 124.46 106.68) (end 127 106.68) (width 1) (layer B.Cu) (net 7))
 (segment (start 148.59 100.33) (end 149.86 99.06) (width 1) (layer B.Cu) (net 7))
 (segment (start 148.59 101.6) (end 148.59 100.33) (width 1) (layer B.Cu) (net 7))
 (segment (start 151.13 104.14) (end 148.59 101.6) (width 1) (layer B.Cu) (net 7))
 (segment (start 149.86 99.06) (end 149.86 97.79) (width 0.5) (layer B.Cu) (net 7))
 (segment (start 149.86 97.79) (end 148.044784 95.974784) (width 0.5) (layer B.Cu) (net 7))
 (via (at 138.43 124.46) (size 1.4) (drill 0.8) (layers F.Cu B.Cu) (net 7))
 (segment (start 161.29 104.14) (end 163.195 104.14) (width 1) (layer B.Cu) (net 7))
 (segment (start 145.482919 90.805) (end 147.955 90.805) (width 1) (layer B.Cu) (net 7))
 (segment (start 144.78 88.9) (end 144.78 90.102081) (width 1) (layer B.Cu) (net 7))
 (segment (start 144.78 90.102081) (end 145.482919 90.805) (width 1) (layer B.Cu) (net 7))
 (segment (start 122.618001 107.251999) (end 123.19 106.68) (width 1) (layer B.Cu) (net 7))
 (segment (start 126.332451 112.395) (end 126.332451 112.395) (width 1) (layer B.Cu) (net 7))
 (segment (start 142.24 125.73) (end 140.97 124.46) (width 1) (layer B.Cu) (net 7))
 (segment (start 123.19 106.68) (end 124.46 106.68) (width 1) (layer B.Cu) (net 7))
 (segment (start 142.24 127) (end 142.24 125.73) (width 1) (layer B.Cu) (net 7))
 (segment (start 122.618001 111.188001) (end 122.618001 107.251999) (width 1) (layer B.Cu) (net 7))
 (segment (start 132.715 124.46) (end 127.635 119.38) (width 1) (layer B.Cu) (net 7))
 (segment (start 123.825 112.395) (end 122.618001 111.188001) (width 1) (layer B.Cu) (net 7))
 (segment (start 140.97 124.46) (end 132.715 124.46) (width 1) (layer B.Cu) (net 7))
 (segment (start 138.43 124.46) (end 156.845 106.045) (width 1) (layer F.Cu) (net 7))
 (segment (start 156.845 106.045) (end 156.845 106.045) (width 1) (layer F.Cu) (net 7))
 (via (at 156.845 106.045) (size 1.4) (drill 0.8) (layers F.Cu B.Cu) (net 7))
 (segment (start 160.02 109.22) (end 156.845 106.045) (width 1) (layer B.Cu) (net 7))
 (segment (start 162.56 109.22) (end 160.02 109.22) (width 1) (layer B.Cu) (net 7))
 (segment (start 156.845 106.045) (end 154.94 104.14) (width 1) (layer B.Cu) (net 7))
 (segment (start 154.94 104.14) (end 151.13 104.14) (width 1) (layer B.Cu) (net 7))
 (segment (start 126.332451 112.395) (end 123.825 112.395) (width 1) (layer B.Cu) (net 7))
 (via (at 126.332451 112.395) (size 1.4) (drill 0.8) (layers F.Cu B.Cu) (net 7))
 (segment (start 147.955 90.805) (end 149.225 92.075) (width 1) (layer B.Cu) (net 7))
 (segment (start 149.225 92.075) (end 161.29 104.14) (width 1) (layer B.Cu) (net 7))
 (via (at 149.225 92.075) (size 1.4) (drill 0.8) (layers F.Cu B.Cu) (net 7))
 (segment (start 127 118.745) (end 132.715 124.46) (width 1) (layer B.Cu) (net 7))
 (segment (start 127 113.062549) (end 127 118.745) (width 1) (layer B.Cu) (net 7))
 (segment (start 127 113.062549) (end 126.332451 112.395) (width 1) (layer B.Cu) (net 7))
 (segment (start 129.231847 104.448153) (end 128.27 103.486306) (width 1) (layer F.Cu) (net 7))
 (segment (start 128.27 103.486306) (end 128.27 102.235) (width 1) (layer F.Cu) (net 7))
 (segment (start 128.27 102.235) (end 139.7 90.805) (width 1) (layer F.Cu) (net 7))
 (segment (start 139.7 90.805) (end 139.7 88.265) (width 1) (layer F.Cu) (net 7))
 (segment (start 140.715001 87.249999) (end 144.399999 87.249999) (width 1) (layer F.Cu) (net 7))
 (segment (start 139.7 88.265) (end 140.715001 87.249999) (width 1) (layer F.Cu) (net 7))
 (segment (start 144.78 87.63) (end 144.78 88.9) (width 1) (layer F.Cu) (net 7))
 (segment (start 144.399999 87.249999) (end 144.78 87.63) (width 1) (layer F.Cu) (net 7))
 (segment (start 129.54 109.22) (end 130.81 107.95) (width 0.5) (layer B.Cu) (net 5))
 (segment (start 129.54 111.125) (end 129.54 109.22) (width 0.5) (layer B.Cu) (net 5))
 (segment (start 133.985 102.017102) (end 132.823949 100.856051) (width 0.5) (layer B.Cu) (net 5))
 (segment (start 133.985 102.87) (end 133.985 102.017102) (width 0.5) (layer B.Cu) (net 5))
 (segment (start 132.715 104.14) (end 133.985 102.87) (width 0.5) (layer B.Cu) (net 5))
 (segment (start 130.81 107.95) (end 132.715 106.045) (width 0.5) (layer B.Cu) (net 5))
 (segment (start 132.715 106.045) (end 132.715 104.14) (width 0.5) (layer B.Cu) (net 5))
 (segment (start 132.113958 116.998168) (end 132.113958 113.698958) (width 0.5) (layer B.Cu) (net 5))
 (segment (start 131.477563 117.634563) (end 132.113958 116.998168) (width 0.5) (layer B.Cu) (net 5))
 (segment (start 132.081395 113.666395) (end 131.064 112.649) (width 0.5) (layer B.Cu) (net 5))
 (segment (start 131.064 112.649) (end 129.54 111.125) (width 0.5) (layer B.Cu) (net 5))
 (segment (start 145.145648 95.974784) (end 146.595216 94.525216) (width 0.5) (layer B.Cu) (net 2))
 (segment (start 144.869784 95.974784) (end 145.145648 95.974784) (width 0.5) (layer B.Cu) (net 2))
 (segment (start 144.3041 96.540468) (end 144.869784 95.974784) (width 0.5) (layer B.Cu) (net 2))
 (segment (start 144.165468 96.540468) (end 144.3041 96.540468) (width 0.5) (layer B.Cu) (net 2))
 (segment (start 144.145 96.52) (end 144.165468 96.540468) (width 0.5) (layer B.Cu) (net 2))
 (segment (start 139.264206 96.52) (end 144.145 96.52) (width 0.5) (layer B.Cu) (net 2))
 (segment (start 138.212103 95.467897) (end 139.264206 96.52) (width 0.5) (layer B.Cu) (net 2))
 (segment (start 155.992103 113.247897) (end 154.504206 111.76) (width 0.5) (layer B.Cu) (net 9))
 (segment (start 154.504206 111.76) (end 153.035 111.76) (width 0.5) (layer B.Cu) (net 9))
 (segment (start 153.035 111.76) (end 146.05 118.745) (width 0.5) (layer B.Cu) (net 9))
 (segment (start 146.05 118.745) (end 144.78 118.745) (width 0.5) (layer B.Cu) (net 9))
 (segment (start 144.78 118.745) (end 138.43 112.395) (width 0.5) (layer B.Cu) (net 9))
 (segment (start 137.141308 112.395) (end 136.198154 113.338154) (width 0.5) (layer B.Cu) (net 9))
 (segment (start 138.43 112.395) (end 137.141308 112.395) (width 0.5) (layer B.Cu) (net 9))
 (segment (start 141.605 118.745) (end 143.51 120.65) (width 0.5) (layer B.Cu) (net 10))
 (segment (start 137.994205 115.134205) (end 141.605 118.745) (width 0.5) (layer B.Cu) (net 10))
 (segment (start 143.51 120.65) (end 144.78 120.65) (width 0.5) (layer B.Cu) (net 10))
 (segment (start 144.78 120.65) (end 145.415 120.65) (width 0.5) (layer B.Cu) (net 10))
 (segment (start 151.871051 114.193949) (end 150.495 115.57) (width 0.5) (layer B.Cu) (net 10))
 (segment (start 153.346053 114.193949) (end 151.871051 114.193949) (width 0.5) (layer B.Cu) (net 10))
 (segment (start 154.196052 115.043948) (end 153.346053 114.193949) (width 0.5) (layer B.Cu) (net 10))
 (segment (start 145.415 120.65) (end 150.495 115.57) (width 0.5) (layer B.Cu) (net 10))
 (segment (start 150.495 115.57) (end 151.765 114.3) (width 0.5) (layer B.Cu) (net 10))
 (segment (start 158.096308 111.76) (end 157.788154 111.451846) (width 0.5) (layer B.Cu) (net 12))
 (segment (start 162.56 111.76) (end 158.096308 111.76) (width 0.5) (layer B.Cu) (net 12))
 (segment (start 139.7 128.35) (end 140.255 128.905) (width 0.5) (layer B.Cu) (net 11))
 (segment (start 139.7 127) (end 139.7 128.35) (width 0.5) (layer B.Cu) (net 11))
 (segment (start 140.255 128.905) (end 146.685 128.905) (width 0.5) (layer B.Cu) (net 11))
 (segment (start 147.011847 128.578153) (end 147.011847 122.228153) (width 0.5) (layer B.Cu) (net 11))
 (segment (start 146.685 128.905) (end 147.011847 128.578153) (width 0.5) (layer B.Cu) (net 11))
 (segment (start 124.46 104.14) (end 125.81 104.14) (width 0.5) (layer B.Cu) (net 4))
 (segment (start 131.739999 98.210001) (end 130.255 99.695) (width 0.5) (layer B.Cu) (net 4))
 (segment (start 133.770001 98.210001) (end 131.739999 98.210001) (width 0.5) (layer B.Cu) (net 4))
 (segment (start 134.62 99.06) (end 133.770001 98.210001) (width 0.5) (layer B.Cu) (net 4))
 (segment (start 125.81 104.14) (end 130.255 99.695) (width 0.5) (layer B.Cu) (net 4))
 (segment (start 130.255 99.695) (end 131.525 98.425) (width 0.5) (layer B.Cu) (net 4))
 (segment (start 147.32 87.55) (end 147.32 88.9) (width 0.5) (layer B.Cu) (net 1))
 (segment (start 140.008154 93.671846) (end 140.008154 92.369764) (width 0.5) (layer B.Cu) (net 1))
 (segment (start 140.008154 92.369764) (end 139.065 91.42661) (width 0.5) (layer B.Cu) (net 1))
 (segment (start 139.065 91.42661) (end 139.065 88.265) (width 0.5) (layer B.Cu) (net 1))
 (segment (start 139.065 88.265) (end 140.521999 86.808001) (width 0.5) (layer B.Cu) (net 1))
 (segment (start 140.521999 86.808001) (end 146.578001 86.808001) (width 0.5) (layer B.Cu) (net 1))
 (segment (start 146.578001 86.808001) (end 147.32 87.55) (width 0.5) (layer B.Cu) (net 1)))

